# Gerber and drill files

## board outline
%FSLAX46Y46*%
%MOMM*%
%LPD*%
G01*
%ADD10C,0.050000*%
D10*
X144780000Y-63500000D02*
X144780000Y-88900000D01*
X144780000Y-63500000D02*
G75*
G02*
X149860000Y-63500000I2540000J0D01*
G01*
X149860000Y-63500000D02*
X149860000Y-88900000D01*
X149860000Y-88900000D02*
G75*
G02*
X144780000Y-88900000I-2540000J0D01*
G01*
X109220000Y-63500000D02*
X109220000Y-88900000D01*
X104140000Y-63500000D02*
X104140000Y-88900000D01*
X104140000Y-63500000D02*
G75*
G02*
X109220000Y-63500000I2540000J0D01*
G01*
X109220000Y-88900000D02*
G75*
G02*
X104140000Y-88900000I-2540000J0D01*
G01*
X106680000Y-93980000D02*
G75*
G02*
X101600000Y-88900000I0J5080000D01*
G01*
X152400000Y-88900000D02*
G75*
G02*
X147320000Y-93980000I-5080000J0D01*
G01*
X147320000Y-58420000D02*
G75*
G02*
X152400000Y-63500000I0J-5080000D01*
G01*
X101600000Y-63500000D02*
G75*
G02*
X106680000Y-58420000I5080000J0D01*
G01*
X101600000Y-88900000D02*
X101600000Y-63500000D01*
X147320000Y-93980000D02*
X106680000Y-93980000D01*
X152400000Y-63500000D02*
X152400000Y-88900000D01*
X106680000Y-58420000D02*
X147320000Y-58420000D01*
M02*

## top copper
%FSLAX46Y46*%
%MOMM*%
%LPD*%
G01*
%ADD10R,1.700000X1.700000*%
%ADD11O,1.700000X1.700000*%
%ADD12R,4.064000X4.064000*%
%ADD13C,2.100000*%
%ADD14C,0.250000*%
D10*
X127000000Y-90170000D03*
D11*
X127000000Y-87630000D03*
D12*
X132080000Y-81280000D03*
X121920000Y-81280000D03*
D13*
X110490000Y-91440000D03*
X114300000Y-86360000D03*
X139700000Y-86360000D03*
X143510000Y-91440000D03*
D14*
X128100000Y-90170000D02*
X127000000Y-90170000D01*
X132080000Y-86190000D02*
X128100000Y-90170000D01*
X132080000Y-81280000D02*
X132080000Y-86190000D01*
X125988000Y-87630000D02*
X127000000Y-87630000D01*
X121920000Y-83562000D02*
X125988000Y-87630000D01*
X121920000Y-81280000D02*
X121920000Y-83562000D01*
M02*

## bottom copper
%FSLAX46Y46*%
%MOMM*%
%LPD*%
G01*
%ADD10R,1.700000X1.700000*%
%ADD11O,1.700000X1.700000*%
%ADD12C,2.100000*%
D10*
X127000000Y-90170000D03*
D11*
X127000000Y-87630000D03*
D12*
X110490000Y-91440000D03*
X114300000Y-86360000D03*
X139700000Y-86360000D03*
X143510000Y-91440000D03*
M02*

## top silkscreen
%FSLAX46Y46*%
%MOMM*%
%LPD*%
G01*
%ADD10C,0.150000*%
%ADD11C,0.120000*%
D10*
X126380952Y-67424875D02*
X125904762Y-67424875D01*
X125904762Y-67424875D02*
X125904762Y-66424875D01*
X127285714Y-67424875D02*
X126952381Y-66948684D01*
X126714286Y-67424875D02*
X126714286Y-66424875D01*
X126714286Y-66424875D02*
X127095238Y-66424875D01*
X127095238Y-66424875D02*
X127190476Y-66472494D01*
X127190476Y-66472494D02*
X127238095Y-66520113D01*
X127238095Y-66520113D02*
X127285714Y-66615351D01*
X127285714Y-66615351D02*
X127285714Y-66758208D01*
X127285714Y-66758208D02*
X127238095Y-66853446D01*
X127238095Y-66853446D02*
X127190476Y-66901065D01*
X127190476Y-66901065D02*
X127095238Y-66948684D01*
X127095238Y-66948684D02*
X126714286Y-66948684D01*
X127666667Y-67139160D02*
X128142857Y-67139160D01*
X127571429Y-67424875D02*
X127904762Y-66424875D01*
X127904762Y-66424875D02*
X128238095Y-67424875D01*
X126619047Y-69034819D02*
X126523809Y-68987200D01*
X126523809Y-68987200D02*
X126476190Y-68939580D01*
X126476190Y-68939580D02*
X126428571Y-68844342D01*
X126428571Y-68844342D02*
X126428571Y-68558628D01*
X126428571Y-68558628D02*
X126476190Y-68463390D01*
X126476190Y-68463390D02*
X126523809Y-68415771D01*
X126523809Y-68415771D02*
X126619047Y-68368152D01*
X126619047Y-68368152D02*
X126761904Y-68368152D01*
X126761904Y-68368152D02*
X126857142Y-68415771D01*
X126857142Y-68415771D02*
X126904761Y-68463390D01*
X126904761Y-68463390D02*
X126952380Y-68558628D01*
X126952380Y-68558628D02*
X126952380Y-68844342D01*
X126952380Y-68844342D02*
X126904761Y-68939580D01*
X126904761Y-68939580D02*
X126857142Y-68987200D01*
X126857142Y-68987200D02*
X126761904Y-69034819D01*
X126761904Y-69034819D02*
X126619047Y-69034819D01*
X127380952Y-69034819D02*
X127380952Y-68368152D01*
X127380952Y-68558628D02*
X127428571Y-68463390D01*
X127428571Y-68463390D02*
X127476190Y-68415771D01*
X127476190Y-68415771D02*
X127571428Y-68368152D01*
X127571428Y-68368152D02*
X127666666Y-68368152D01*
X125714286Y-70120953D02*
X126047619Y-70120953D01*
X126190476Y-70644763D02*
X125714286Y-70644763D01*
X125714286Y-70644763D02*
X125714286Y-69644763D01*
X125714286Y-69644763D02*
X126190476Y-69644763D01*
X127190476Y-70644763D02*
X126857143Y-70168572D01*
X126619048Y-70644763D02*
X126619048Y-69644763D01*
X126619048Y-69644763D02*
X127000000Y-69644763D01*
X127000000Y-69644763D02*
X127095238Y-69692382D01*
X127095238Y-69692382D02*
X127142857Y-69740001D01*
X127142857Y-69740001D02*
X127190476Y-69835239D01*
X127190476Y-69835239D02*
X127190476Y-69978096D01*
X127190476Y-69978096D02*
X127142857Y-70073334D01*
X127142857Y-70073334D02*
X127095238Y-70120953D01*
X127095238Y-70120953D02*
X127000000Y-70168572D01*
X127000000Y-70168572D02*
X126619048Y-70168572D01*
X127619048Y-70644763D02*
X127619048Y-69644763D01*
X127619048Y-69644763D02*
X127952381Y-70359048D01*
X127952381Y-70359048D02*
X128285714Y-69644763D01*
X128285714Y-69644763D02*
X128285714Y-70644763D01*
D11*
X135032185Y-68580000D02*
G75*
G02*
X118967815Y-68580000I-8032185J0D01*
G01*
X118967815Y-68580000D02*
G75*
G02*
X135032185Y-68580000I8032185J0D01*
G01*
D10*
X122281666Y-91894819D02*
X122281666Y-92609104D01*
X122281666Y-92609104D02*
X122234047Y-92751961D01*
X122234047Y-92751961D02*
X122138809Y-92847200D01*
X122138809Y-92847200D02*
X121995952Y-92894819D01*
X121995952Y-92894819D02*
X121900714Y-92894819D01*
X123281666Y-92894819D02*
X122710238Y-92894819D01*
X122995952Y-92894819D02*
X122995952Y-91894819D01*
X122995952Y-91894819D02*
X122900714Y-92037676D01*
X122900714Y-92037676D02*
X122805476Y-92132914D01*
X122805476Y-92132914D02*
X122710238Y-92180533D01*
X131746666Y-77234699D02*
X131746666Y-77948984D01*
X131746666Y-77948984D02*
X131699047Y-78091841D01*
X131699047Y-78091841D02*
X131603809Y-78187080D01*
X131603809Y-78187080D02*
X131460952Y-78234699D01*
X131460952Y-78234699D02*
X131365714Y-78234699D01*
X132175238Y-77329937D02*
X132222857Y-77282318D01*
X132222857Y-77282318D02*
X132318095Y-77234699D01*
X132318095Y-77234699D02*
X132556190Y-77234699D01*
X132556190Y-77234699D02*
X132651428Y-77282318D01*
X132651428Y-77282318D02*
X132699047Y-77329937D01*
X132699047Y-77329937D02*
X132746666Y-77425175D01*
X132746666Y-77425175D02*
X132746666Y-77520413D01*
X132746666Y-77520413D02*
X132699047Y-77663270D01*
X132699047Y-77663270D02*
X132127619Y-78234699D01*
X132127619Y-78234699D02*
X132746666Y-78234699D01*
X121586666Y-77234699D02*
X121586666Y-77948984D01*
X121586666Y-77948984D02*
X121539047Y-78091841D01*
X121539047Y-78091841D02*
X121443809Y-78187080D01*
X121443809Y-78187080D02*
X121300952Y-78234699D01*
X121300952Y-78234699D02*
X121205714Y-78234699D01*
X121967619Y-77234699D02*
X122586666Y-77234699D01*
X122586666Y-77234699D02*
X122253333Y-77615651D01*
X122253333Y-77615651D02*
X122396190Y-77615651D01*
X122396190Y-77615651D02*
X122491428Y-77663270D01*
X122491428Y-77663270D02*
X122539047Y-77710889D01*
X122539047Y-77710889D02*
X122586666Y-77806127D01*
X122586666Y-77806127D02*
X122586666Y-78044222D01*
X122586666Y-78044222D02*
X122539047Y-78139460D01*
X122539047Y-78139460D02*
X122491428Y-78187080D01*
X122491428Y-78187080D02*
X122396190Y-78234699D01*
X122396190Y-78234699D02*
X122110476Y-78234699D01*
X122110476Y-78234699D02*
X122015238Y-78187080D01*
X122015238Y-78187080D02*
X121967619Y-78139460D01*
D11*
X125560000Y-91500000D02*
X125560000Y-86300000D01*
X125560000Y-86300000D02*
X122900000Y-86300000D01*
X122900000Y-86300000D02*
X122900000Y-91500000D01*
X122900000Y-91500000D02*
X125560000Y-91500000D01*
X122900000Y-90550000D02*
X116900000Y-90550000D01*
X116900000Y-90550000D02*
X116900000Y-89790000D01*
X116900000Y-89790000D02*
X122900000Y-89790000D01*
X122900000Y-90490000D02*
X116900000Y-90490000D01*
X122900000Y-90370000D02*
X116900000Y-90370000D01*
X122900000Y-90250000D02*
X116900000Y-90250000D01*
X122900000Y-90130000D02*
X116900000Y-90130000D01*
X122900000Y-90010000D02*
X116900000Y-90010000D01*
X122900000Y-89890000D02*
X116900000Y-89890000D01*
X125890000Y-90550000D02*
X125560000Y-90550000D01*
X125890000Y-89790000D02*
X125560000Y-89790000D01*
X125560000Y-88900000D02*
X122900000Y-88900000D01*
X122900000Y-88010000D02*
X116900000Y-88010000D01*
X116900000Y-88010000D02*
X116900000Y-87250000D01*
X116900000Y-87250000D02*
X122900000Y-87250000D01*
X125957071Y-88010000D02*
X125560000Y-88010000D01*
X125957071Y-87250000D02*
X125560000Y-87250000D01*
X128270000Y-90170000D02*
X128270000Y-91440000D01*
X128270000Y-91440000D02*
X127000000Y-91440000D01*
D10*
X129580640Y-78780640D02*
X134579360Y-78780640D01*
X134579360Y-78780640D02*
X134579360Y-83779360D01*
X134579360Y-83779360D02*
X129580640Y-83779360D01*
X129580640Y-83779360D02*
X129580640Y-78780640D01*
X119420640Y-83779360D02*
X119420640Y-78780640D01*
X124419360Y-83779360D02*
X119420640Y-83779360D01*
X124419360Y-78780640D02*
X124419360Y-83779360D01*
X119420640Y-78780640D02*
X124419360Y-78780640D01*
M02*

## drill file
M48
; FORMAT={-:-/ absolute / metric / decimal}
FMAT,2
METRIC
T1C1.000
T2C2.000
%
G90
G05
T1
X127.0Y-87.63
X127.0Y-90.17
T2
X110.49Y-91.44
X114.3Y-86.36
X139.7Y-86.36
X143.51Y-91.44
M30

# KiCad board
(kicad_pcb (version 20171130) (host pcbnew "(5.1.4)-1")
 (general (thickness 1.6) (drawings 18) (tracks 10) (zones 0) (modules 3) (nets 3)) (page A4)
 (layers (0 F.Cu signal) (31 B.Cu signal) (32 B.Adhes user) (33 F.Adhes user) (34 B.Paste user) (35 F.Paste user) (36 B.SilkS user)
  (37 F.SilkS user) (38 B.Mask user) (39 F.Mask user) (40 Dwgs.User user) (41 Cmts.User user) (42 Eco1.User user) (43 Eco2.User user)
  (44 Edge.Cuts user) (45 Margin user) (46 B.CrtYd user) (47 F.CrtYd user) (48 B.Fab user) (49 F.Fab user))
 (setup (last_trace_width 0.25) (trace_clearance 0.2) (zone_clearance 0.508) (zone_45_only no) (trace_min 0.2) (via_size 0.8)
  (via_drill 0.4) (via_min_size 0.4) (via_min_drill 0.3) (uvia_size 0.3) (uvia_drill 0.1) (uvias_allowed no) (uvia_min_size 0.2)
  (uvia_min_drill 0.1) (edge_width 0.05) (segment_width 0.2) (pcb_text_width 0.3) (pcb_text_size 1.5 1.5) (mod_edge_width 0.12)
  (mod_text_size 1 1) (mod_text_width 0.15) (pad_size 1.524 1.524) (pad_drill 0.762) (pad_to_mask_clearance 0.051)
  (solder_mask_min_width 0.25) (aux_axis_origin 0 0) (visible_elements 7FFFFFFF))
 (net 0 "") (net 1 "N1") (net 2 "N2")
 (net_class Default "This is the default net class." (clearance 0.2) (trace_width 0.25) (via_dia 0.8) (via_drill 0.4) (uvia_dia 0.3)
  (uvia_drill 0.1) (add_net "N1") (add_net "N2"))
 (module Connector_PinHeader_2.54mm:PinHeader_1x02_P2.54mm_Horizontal (layer F.Cu) (at 127 90.17 180)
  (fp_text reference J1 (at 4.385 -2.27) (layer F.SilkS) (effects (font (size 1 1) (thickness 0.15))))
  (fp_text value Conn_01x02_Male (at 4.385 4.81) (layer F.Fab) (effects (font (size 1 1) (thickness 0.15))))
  (fp_line (start 1.44 -1.33) (end 1.44 3.87) (layer F.SilkS) (width 0.12))
  (fp_line (start 1.44 3.87) (end 4.1 3.87) (layer F.SilkS) (width 0.12))
  (fp_line (start 4.1 3.87) (end 4.1 -1.33) (layer F.SilkS) (width 0.12))
  (fp_line (start 4.1 -1.33) (end 1.44 -1.33) (layer F.SilkS) (width 0.12))
  (fp_line (start 4.1 -0.38) (end 10.1 -0.38) (layer F.SilkS) (width 0.12))
  (fp_line (start 10.1 -0.38) (end 10.1 0.38) (layer F.SilkS) (width 0.12))
  (fp_line (start 10.1 0.38) (end 4.1 0.38) (layer F.SilkS) (width 0.12))
  (fp_line (start 4.1 -0.32) (end 10.1 -0.32) (layer F.SilkS) (width 0.12))
  (fp_line (start 4.1 -0.2) (end 10.1 -0.2) (layer F.SilkS) (width 0.12))
  (fp_line (start 4.1 -0.08) (end 10.1 -0.08) (layer F.SilkS) (width 0.12))
  (fp_line (start 4.1 0.04) (end 10.1 0.04) (layer F.SilkS) (width 0.12))
  (fp_line (start 4.1 0.16) (end 10.1 0.16) (layer F.SilkS) (width 0.12))
  (fp_line (start 4.1 0.28) (end 10.1 0.28) (layer F.SilkS) (width 0.12))
  (fp_line (start 1.11 -0.38) (end 1.44 -0.38) (layer F.SilkS) (width 0.12))
  (fp_line (start 1.11 0.38) (end 1.44 0.38) (layer F.SilkS) (width 0.12))
  (fp_line (start 1.44 1.27) (end 4.1 1.27) (layer F.SilkS) (width 0.12))
  (fp_line (start 4.1 2.16) (end 10.1 2.16) (layer F.SilkS) (width 0.12))
  (fp_line (start 10.1 2.16) (end 10.1 2.92) (layer F.SilkS) (width 0.12))
  (fp_line (start 10.1 2.92) (end 4.1 2.92) (layer F.SilkS) (width 0.12))
  (fp_line (start 1.042929 2.16) (end 1.44 2.16) (layer F.SilkS) (width 0.12))
  (fp_line (start 1.042929 2.92) (end 1.44 2.92) (layer F.SilkS) (width 0.12))
  (fp_line (start -1.27 0) (end -1.27 -1.27) (layer F.SilkS) (width 0.12))
  (fp_line (start -1.27 -1.27) (end 0 -1.27) (layer F.SilkS) (width 0.12))
  (pad 1 thru_hole rect (at 0 0 180) (size 1.7 1.7) (drill 1) (layers *.Cu *.Mask) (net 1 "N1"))
  (pad 2 thru_hole oval (at 0 2.54 180) (size 1.7 1.7) (drill 1) (layers *.Cu *.Mask) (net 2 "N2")))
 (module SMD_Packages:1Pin (layer F.Cu) (at 132.08 81.28)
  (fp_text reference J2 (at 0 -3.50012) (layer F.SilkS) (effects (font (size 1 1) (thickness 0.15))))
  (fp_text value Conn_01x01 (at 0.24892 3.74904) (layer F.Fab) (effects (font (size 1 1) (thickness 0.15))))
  (fp_line (start -2.49936 -2.49936) (end 2.49936 -2.49936) (layer F.SilkS) (width 0.15))
  (fp_line (start 2.49936 -2.49936) (end 2.49936 2.49936) (layer F.SilkS) (width 0.15))
  (fp_line (start 2.49936 2.49936) (end -2.49936 2.49936) (layer F.SilkS) (width 0.15))
  (fp_line (start -2.49936 2.49936) (end -2.49936 -2.49936) (layer F.SilkS) (width 0.15))
  (pad 1 smd rect (at 0 0) (size 4.064 4.064) (layers F.Cu F.Paste F.Mask) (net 1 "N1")))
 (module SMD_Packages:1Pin (layer F.Cu) (at 121.92 81.28)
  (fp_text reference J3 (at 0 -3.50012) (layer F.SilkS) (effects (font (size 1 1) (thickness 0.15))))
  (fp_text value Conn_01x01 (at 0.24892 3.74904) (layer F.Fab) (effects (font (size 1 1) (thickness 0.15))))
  (fp_line (start -2.49936 2.49936) (end -2.49936 -2.49936) (layer F.SilkS) (width 0.15))
  (fp_line (start 2.49936 2.49936) (end -2.49936 2.49936) (layer F.SilkS) (width 0.15))
  (fp_line (start 2.49936 -2.49936) (end 2.49936 2.49936) (layer F.SilkS) (width 0.15))
  (fp_line (start -2.49936 -2.49936) (end 2.49936 -2.49936) (layer F.SilkS) (width 0.15))
  (pad 1 smd rect (at 0 0) (size 4.064 4.064) (layers F.Cu F.Paste F.Mask) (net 2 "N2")))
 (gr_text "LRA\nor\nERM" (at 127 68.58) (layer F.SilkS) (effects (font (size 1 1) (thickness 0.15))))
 (gr_circle (center 127 68.58) (end 134.62 71.12) (layer F.SilkS) (width 0.12))
 (gr_line (start 144.78 63.5) (end 144.78 88.9) (layer Edge.Cuts) (width 0.05))
 (gr_arc (start 147.32 63.5) (end 149.86 63.5) (angle -180) (layer Edge.Cuts) (width 0.05))
 (gr_line (start 149.86 63.5) (end 149.86 88.9) (layer Edge.Cuts) (width 0.05))
 (gr_arc (start 147.32 88.9) (end 144.78 88.9) (angle -180) (layer Edge.Cuts) (width 0.05))
 (gr_line (start 109.22 63.5) (end 109.22 88.9) (layer Edge.Cuts) (width 0.05))
 (gr_line (start 104.14 63.5) (end 104.14 88.9) (layer Edge.Cuts) (width 0.05))
 (gr_arc (start 106.68 63.5) (end 109.22 63.5) (angle -180) (layer Edge.Cuts) (width 0.05))
 (gr_arc (start 106.68 88.9) (end 104.14 88.9) (angle -180) (layer Edge.Cuts) (width 0.05))
 (gr_arc (start 106.68 88.9) (end 101.6 88.9) (angle -90) (layer Edge.Cuts) (width 0.05))
 (gr_arc (start 147.32 88.9) (end 147.32 93.98) (angle -90) (layer Edge.Cuts) (width 0.05))
 (gr_arc (start 147.32 63.5) (end 152.4 63.5) (angle -90) (layer Edge.Cuts) (width 0.05))
 (gr_arc (start 106.68 63.5) (end 106.68 58.42) (angle -90) (layer Edge.Cuts) (width 0.05))
 (gr_line (start 101.6 88.9) (end 101.6 63.5) (layer Edge.Cuts) (width 0.05))
 (gr_line (start 147.32 93.98) (end 106.68 93.98) (layer Edge.Cuts) (width 0.05))
 (gr_line (start 152.4 63.5) (end 152.4 88.9) (layer Edge.Cuts) (width 0.05))
 (gr_line (start 106.68 58.42) (end 147.32 58.42) (layer Edge.Cuts) (width 0.05))
 (via (at 110.49 91.44) (size 2.1) (drill 2) (layers F.Cu B.Cu) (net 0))
 (via (at 114.3 86.36) (size 2.1) (drill 2) (layers F.Cu B.Cu) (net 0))
 (via (at 139.7 86.36) (size 2.1) (drill 2) (layers F.Cu B.Cu) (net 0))
 (via (at 143.51 91.44) (size 2.1) (drill 2) (layers F.Cu B.Cu) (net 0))
 (segment (start 128.1 90.17) (end 127 90.17) (width 0.25) (layer F.Cu) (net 1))
 (segment (start 132.08 86.19) (end 128.1 90.17) (width 0.25) (layer F.Cu) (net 1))
 (segment (start 132.08 81.28) (end 132.08 86.19) (width 0.25) (layer F.Cu) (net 1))
 (segment (start 125.988 87.63) (end 127 87.63) (width 0.25) (layer F.Cu) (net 2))
 (segment (start 121.92 83.562) (end 125.988 87.63) (width 0.25) (layer F.Cu) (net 2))
 (segment (start 121.92 81.28) (end 121.92 83.562) (width 0.25) (layer F.Cu) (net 2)))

